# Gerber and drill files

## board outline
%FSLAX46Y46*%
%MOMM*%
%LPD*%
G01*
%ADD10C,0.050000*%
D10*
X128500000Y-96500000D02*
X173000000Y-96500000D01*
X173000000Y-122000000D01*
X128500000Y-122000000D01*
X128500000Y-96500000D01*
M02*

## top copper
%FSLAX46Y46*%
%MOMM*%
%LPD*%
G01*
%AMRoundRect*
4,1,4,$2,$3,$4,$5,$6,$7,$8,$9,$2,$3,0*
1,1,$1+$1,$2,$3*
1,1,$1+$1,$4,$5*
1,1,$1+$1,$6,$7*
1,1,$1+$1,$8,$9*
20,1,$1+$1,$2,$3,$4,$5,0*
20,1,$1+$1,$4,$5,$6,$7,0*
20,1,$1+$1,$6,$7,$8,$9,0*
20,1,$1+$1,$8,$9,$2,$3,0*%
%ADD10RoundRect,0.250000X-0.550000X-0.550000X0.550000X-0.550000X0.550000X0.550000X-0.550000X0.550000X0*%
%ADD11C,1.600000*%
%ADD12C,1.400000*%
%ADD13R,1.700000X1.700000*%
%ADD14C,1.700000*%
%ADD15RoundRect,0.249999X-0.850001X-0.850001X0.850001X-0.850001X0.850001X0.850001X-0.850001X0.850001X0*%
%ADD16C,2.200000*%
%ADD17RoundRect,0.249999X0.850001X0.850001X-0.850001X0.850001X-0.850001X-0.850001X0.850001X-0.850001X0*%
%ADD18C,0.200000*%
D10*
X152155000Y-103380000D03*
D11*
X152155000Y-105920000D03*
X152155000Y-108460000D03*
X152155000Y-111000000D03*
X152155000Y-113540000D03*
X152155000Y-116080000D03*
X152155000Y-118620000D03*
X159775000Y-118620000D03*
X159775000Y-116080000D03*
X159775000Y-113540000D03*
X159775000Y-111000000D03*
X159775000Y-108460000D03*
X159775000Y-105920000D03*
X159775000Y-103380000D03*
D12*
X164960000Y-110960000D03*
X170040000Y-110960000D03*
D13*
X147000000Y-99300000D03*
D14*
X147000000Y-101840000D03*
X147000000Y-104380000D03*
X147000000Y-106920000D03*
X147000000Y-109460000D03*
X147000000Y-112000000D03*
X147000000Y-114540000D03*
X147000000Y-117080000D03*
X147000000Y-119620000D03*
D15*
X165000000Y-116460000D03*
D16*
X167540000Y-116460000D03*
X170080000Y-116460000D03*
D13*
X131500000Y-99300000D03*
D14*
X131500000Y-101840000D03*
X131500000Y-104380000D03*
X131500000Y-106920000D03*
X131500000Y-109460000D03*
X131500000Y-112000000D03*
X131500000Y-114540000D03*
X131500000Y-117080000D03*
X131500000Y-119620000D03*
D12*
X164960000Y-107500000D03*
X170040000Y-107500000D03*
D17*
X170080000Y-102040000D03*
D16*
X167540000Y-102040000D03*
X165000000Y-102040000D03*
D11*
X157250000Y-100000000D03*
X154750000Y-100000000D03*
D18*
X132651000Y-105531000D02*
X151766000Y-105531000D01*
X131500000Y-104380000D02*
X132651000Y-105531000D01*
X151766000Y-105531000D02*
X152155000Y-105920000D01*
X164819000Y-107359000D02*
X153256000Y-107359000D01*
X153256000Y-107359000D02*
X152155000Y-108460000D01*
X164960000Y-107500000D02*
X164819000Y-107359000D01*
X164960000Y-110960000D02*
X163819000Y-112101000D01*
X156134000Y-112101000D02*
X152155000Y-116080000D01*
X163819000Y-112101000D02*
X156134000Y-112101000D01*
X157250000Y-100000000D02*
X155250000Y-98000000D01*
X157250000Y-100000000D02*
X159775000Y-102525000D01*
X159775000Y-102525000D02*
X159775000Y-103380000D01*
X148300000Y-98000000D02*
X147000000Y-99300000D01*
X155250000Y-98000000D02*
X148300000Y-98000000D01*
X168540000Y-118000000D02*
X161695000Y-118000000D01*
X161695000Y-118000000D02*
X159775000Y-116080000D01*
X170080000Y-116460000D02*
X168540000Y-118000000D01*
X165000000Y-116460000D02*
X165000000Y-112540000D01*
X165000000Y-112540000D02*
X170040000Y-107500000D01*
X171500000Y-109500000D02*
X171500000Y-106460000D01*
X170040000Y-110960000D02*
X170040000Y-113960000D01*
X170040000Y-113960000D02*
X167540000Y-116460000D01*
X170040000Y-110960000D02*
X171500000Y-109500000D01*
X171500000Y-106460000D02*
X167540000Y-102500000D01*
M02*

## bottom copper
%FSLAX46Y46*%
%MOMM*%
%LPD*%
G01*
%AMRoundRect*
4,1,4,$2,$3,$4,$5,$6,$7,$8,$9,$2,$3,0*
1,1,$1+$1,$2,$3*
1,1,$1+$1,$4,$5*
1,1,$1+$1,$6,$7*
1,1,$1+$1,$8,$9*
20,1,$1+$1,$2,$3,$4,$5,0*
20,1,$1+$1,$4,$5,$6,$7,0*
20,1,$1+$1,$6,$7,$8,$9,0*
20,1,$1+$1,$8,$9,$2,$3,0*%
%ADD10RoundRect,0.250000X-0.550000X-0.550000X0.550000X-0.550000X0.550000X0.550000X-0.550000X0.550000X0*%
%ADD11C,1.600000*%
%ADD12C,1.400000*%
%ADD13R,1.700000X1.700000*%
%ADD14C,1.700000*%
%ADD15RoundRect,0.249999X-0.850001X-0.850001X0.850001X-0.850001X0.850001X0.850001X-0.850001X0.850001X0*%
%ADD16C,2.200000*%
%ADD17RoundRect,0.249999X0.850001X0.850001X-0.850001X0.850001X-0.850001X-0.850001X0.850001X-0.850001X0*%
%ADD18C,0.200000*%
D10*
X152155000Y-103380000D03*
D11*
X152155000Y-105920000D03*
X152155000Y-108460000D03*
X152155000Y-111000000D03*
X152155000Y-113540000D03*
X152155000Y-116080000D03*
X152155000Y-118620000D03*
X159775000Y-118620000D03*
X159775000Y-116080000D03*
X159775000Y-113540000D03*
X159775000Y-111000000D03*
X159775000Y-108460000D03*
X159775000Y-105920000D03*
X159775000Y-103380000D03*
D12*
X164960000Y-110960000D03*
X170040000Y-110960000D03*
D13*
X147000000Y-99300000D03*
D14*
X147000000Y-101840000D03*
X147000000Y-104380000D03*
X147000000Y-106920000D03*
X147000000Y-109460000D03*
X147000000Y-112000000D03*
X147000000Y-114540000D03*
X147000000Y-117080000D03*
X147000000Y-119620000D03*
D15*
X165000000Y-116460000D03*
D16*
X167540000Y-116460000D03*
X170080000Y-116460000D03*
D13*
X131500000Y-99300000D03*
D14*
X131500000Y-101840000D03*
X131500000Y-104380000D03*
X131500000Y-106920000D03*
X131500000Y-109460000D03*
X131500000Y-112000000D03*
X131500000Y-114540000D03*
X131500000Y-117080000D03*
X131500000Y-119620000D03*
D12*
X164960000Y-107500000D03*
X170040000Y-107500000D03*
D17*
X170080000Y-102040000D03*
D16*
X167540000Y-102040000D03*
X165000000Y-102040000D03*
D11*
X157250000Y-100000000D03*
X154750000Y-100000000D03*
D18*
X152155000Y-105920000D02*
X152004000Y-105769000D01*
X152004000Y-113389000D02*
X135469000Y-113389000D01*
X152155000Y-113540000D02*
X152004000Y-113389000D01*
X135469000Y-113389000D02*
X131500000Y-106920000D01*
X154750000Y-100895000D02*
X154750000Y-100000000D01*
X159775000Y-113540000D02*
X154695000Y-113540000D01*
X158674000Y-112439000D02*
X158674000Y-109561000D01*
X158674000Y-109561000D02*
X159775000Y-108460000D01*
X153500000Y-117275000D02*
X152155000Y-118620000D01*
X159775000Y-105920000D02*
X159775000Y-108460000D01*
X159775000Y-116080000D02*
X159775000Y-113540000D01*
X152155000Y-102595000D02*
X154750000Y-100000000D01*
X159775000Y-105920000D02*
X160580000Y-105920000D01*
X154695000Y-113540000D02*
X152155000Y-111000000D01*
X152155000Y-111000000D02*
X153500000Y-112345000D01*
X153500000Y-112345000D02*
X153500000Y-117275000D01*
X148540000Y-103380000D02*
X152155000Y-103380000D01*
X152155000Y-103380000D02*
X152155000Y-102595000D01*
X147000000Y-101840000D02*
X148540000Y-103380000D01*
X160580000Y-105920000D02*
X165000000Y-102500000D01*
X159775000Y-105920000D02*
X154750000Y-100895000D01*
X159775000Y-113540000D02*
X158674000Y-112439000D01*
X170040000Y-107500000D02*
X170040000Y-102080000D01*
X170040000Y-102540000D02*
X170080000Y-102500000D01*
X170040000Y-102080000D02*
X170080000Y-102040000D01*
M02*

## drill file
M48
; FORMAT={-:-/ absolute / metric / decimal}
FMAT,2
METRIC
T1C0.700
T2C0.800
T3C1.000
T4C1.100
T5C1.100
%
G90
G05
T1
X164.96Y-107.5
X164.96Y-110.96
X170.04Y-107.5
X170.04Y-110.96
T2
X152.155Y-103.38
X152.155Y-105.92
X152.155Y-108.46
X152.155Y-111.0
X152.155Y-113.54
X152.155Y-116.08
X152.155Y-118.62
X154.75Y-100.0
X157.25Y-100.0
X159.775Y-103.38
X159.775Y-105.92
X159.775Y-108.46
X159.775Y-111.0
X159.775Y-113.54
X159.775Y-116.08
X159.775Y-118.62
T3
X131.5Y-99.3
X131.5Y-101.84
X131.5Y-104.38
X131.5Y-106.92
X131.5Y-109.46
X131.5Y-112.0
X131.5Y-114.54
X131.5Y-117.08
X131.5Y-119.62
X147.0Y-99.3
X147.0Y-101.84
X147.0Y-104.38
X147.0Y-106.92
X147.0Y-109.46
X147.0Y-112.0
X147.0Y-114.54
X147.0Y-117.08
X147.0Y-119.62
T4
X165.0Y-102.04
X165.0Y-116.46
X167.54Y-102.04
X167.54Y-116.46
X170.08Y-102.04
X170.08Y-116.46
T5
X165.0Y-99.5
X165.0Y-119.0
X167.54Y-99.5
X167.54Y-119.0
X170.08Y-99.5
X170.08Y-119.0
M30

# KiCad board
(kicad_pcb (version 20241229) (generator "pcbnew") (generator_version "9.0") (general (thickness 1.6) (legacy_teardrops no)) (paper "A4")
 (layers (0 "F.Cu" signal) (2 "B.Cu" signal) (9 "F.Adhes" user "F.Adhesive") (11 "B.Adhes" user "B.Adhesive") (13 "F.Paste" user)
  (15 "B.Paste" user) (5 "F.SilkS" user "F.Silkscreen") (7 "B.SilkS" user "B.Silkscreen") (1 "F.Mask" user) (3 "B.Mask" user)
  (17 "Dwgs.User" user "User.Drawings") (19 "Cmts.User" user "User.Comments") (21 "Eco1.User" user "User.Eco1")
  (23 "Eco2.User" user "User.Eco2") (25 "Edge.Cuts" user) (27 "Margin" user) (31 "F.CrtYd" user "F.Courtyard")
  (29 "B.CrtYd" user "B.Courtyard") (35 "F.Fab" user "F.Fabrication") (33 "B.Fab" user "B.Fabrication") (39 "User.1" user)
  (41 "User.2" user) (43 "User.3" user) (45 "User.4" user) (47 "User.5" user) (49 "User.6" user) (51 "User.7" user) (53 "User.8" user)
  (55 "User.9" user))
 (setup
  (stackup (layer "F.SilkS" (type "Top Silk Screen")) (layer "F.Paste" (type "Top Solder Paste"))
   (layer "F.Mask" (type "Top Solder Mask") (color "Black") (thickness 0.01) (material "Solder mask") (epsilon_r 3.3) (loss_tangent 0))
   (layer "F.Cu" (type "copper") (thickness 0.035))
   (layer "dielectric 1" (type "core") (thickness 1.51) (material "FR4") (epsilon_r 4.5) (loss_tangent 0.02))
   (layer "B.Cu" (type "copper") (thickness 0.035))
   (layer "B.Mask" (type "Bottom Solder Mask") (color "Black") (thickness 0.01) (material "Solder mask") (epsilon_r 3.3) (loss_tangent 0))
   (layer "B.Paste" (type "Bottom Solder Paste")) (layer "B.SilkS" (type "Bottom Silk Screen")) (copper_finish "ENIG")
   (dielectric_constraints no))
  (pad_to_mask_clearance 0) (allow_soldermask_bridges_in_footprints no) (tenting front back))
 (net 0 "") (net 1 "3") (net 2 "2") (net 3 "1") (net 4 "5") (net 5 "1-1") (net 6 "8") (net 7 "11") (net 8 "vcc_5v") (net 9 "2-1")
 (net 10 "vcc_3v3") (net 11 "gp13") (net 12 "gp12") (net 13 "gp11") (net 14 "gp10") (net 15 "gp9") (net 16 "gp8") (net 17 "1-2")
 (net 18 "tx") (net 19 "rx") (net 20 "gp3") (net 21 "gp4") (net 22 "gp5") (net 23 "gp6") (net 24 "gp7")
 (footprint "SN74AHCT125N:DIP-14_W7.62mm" (layer "F.Cu") (at 152.155 103.38)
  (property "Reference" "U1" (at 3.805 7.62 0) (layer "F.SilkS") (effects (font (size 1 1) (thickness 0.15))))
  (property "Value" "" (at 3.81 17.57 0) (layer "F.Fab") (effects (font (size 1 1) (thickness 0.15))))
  (pad "1" thru_hole roundrect (at 0 0) (size 1.6 1.6) (drill 0.8) (layers "*.Cu" "*.Mask") (remove_unused_layers no)
   (roundrect_rratio 0.15625) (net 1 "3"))
  (pad "2" thru_hole circle (at 0 2.54) (size 1.6 1.6) (drill 0.8) (layers "*.Cu" "*.Mask") (remove_unused_layers no) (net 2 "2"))
  (pad "3" thru_hole circle (at 0 5.08) (size 1.6 1.6) (drill 0.8) (layers "*.Cu" "*.Mask") (remove_unused_layers no) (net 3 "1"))
  (pad "4" thru_hole circle (at 0 7.62) (size 1.6 1.6) (drill 0.8) (layers "*.Cu" "*.Mask") (remove_unused_layers no) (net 1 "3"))
  (pad "5" thru_hole circle (at 0 10.16) (size 1.6 1.6) (drill 0.8) (layers "*.Cu" "*.Mask") (remove_unused_layers no) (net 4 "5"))
  (pad "6" thru_hole circle (at 0 12.7) (size 1.6 1.6) (drill 0.8) (layers "*.Cu" "*.Mask") (remove_unused_layers no) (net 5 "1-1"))
  (pad "7" thru_hole circle (at 0 15.24) (size 1.6 1.6) (drill 0.8) (layers "*.Cu" "*.Mask") (remove_unused_layers no) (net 1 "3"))
  (pad "8" thru_hole circle (at 7.62 15.24) (size 1.6 1.6) (drill 0.8) (layers "*.Cu" "*.Mask") (remove_unused_layers no) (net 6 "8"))
  (pad "9" thru_hole circle (at 7.62 12.7) (size 1.6 1.6) (drill 0.8) (layers "*.Cu" "*.Mask") (remove_unused_layers no) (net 1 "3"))
  (pad "10" thru_hole circle (at 7.62 10.16) (size 1.6 1.6) (drill 0.8) (layers "*.Cu" "*.Mask") (remove_unused_layers no) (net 1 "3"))
  (pad "11" thru_hole circle (at 7.62 7.62) (size 1.6 1.6) (drill 0.8) (layers "*.Cu" "*.Mask") (remove_unused_layers no) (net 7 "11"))
  (pad "12" thru_hole circle (at 7.62 5.08) (size 1.6 1.6) (drill 0.8) (layers "*.Cu" "*.Mask") (remove_unused_layers no) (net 1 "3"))
  (pad "13" thru_hole circle (at 7.62 2.54) (size 1.6 1.6) (drill 0.8) (layers "*.Cu" "*.Mask") (remove_unused_layers no) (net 1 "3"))
  (pad "14" thru_hole circle (at 7.62 0) (size 1.6 1.6) (drill 0.8) (layers "*.Cu" "*.Mask") (remove_unused_layers no) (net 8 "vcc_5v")))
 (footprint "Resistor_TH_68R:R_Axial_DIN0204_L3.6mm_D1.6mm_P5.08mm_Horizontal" (layer "F.Cu") (at 164.96 110.96)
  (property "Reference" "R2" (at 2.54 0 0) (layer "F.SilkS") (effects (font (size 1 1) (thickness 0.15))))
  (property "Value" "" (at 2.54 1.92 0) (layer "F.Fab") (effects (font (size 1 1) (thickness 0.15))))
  (pad "1" thru_hole circle (at 0 0) (size 1.4 1.4) (drill 0.7) (layers "*.Cu" "*.Mask") (remove_unused_layers no) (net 5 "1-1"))
  (pad "2" thru_hole circle (at 5.08 0) (size 1.4 1.4) (drill 0.7) (layers "*.Cu" "*.Mask") (remove_unused_layers no) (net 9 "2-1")))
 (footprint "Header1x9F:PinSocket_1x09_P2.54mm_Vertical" (layer "F.Cu") (at 147 99.3)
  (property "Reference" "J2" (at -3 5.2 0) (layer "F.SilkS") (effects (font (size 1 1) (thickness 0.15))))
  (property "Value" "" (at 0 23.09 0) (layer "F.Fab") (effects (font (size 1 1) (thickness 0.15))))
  (pad "1" thru_hole rect (at 0 0) (size 1.7 1.7) (drill 1) (layers "*.Cu" "*.Mask") (remove_unused_layers no) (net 8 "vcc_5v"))
  (pad "2" thru_hole circle (at 0 2.54) (size 1.7 1.7) (drill 1) (layers "*.Cu" "*.Mask") (remove_unused_layers no) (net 1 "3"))
  (pad "3" thru_hole circle (at 0 5.08) (size 1.7 1.7) (drill 1) (layers "*.Cu" "*.Mask") (remove_unused_layers no) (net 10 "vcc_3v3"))
  (pad "4" thru_hole circle (at 0 7.62) (size 1.7 1.7) (drill 1) (layers "*.Cu" "*.Mask") (remove_unused_layers no) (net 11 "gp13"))
  (pad "5" thru_hole circle (at 0 10.16) (size 1.7 1.7) (drill 1) (layers "*.Cu" "*.Mask") (remove_unused_layers no) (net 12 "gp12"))
  (pad "6" thru_hole circle (at 0 12.7) (size 1.7 1.7) (drill 1) (layers "*.Cu" "*.Mask") (remove_unused_layers no) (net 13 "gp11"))
  (pad "7" thru_hole circle (at 0 15.24) (size 1.7 1.7) (drill 1) (layers "*.Cu" "*.Mask") (remove_unused_layers no) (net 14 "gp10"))
  (pad "8" thru_hole circle (at 0 17.78) (size 1.7 1.7) (drill 1) (layers "*.Cu" "*.Mask") (remove_unused_layers no) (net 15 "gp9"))
  (pad "9" thru_hole circle (at 0 20.32) (size 1.7 1.7) (drill 1) (layers "*.Cu" "*.Mask") (remove_unused_layers no) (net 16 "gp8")))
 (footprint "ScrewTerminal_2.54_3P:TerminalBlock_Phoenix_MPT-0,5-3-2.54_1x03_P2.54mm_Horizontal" (layer "F.Cu") (at 165 116.46)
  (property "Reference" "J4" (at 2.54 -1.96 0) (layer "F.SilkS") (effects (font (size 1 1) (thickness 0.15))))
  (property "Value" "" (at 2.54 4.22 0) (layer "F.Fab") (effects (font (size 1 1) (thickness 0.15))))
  (pad "" np_thru_hole circle (at 0 2.54) (size 1.1 1.1) (drill 1.1) (layers "*.Cu" "*.Mask"))
  (pad "" np_thru_hole circle (at 2.54 2.54) (size 1.1 1.1) (drill 1.1) (layers "*.Cu" "*.Mask"))
  (pad "" np_thru_hole circle (at 5.08 2.54) (size 1.1 1.1) (drill 1.1) (layers "*.Cu" "*.Mask"))
  (pad "1" thru_hole roundrect (at 0 0) (size 2.2 2.2) (drill 1.1) (layers "*.Cu" "*.Mask") (remove_unused_layers no)
   (roundrect_rratio 0.113636) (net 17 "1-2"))
  (pad "2" thru_hole circle (at 2.54 0) (size 2.2 2.2) (drill 1.1) (layers "*.Cu" "*.Mask") (remove_unused_layers no) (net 9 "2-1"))
  (pad "3" thru_hole circle (at 5.08 0) (size 2.2 2.2) (drill 1.1) (layers "*.Cu" "*.Mask") (remove_unused_layers no) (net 1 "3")))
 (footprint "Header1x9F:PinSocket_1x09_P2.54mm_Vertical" (layer "F.Cu") (at 131.5 99.3)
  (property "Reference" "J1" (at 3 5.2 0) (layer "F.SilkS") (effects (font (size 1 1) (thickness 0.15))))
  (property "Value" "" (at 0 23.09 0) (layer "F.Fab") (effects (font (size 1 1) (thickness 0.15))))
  (pad "1" thru_hole rect (at 0 0) (size 1.7 1.7) (drill 1) (layers "*.Cu" "*.Mask") (remove_unused_layers no) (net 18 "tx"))
  (pad "2" thru_hole circle (at 0 2.54) (size 1.7 1.7) (drill 1) (layers "*.Cu" "*.Mask") (remove_unused_layers no) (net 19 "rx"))
  (pad "3" thru_hole circle (at 0 5.08) (size 1.7 1.7) (drill 1) (layers "*.Cu" "*.Mask") (remove_unused_layers no) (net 2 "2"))
  (pad "4" thru_hole circle (at 0 7.62) (size 1.7 1.7) (drill 1) (layers "*.Cu" "*.Mask") (remove_unused_layers no) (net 4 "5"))
  (pad "5" thru_hole circle (at 0 10.16) (size 1.7 1.7) (drill 1) (layers "*.Cu" "*.Mask") (remove_unused_layers no) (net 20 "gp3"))
  (pad "6" thru_hole circle (at 0 12.7) (size 1.7 1.7) (drill 1) (layers "*.Cu" "*.Mask") (remove_unused_layers no) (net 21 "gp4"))
  (pad "7" thru_hole circle (at 0 15.24) (size 1.7 1.7) (drill 1) (layers "*.Cu" "*.Mask") (remove_unused_layers no) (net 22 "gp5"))
  (pad "8" thru_hole circle (at 0 17.78) (size 1.7 1.7) (drill 1) (layers "*.Cu" "*.Mask") (remove_unused_layers no) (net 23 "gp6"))
  (pad "9" thru_hole circle (at 0 20.32) (size 1.7 1.7) (drill 1) (layers "*.Cu" "*.Mask") (remove_unused_layers no) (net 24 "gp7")))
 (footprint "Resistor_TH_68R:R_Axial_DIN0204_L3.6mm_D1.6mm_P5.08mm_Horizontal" (layer "F.Cu") (at 164.96 107.5)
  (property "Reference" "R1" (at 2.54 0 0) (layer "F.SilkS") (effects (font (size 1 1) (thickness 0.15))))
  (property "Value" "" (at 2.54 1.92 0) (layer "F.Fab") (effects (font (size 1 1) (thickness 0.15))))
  (pad "1" thru_hole circle (at 0 0) (size 1.4 1.4) (drill 0.7) (layers "*.Cu" "*.Mask") (remove_unused_layers no) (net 3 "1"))
  (pad "2" thru_hole circle (at 5.08 0) (size 1.4 1.4) (drill 0.7) (layers "*.Cu" "*.Mask") (remove_unused_layers no) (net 17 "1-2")))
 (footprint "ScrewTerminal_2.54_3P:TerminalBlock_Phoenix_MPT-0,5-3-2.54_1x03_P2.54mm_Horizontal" (layer "F.Cu") (at 170.08 102.04 180)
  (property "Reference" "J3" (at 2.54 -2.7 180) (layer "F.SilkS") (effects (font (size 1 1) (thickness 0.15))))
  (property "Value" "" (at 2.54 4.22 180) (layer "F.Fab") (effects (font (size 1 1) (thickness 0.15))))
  (pad "" np_thru_hole circle (at 0 2.54 180) (size 1.1 1.1) (drill 1.1) (layers "*.Cu" "*.Mask"))
  (pad "" np_thru_hole circle (at 2.54 2.54 180) (size 1.1 1.1) (drill 1.1) (layers "*.Cu" "*.Mask"))
  (pad "" np_thru_hole circle (at 5.08 2.54 180) (size 1.1 1.1) (drill 1.1) (layers "*.Cu" "*.Mask"))
  (pad "1" thru_hole roundrect (at 0 0 180) (size 2.2 2.2) (drill 1.1) (layers "*.Cu" "*.Mask") (remove_unused_layers no)
   (roundrect_rratio 0.113636) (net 17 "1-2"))
  (pad "2" thru_hole circle (at 2.54 0 180) (size 2.2 2.2) (drill 1.1) (layers "*.Cu" "*.Mask") (remove_unused_layers no) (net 9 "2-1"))
  (pad "3" thru_hole circle (at 5.08 0 180) (size 2.2 2.2) (drill 1.1) (layers "*.Cu" "*.Mask") (remove_unused_layers no) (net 1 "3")))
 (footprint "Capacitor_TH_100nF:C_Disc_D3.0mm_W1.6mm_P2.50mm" (layer "F.Cu") (at 157.25 100 180)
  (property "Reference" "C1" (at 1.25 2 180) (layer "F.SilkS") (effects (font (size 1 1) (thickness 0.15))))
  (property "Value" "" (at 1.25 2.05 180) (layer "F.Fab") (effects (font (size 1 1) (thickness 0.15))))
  (pad "1" thru_hole circle (at 0 0 180) (size 1.6 1.6) (drill 0.8) (layers "*.Cu" "*.Mask") (remove_unused_layers no) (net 8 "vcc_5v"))
  (pad "2" thru_hole circle (at 2.5 0 180) (size 1.6 1.6) (drill 0.8) (layers "*.Cu" "*.Mask") (remove_unused_layers no) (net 1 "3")))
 (gr_rect (start 128.5 96.5) (end 173 122) (stroke (width 0.05) (type default)) (fill no) (layer "Edge.Cuts"))
 (segment (start 132.651 105.531) (end 151.766 105.531) (width 0.2) (layer "F.Cu") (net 2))
 (segment (start 131.5 104.38) (end 132.651 105.531) (width 0.2) (layer "F.Cu") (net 2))
 (segment (start 151.766 105.531) (end 152.155 105.92) (width 0.2) (layer "F.Cu") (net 2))
 (segment (start 152.155 105.92) (end 152.004 105.769) (width 0.2) (layer "B.Cu") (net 2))
 (segment (start 152.004 113.389) (end 135.469 113.389) (width 0.2) (layer "B.Cu") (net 4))
 (segment (start 152.155 113.54) (end 152.004 113.389) (width 0.2) (layer "B.Cu") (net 4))
 (segment (start 135.469 113.389) (end 131.5 106.92) (width 0.2) (layer "B.Cu") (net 4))
 (segment (start 164.819 107.359) (end 153.256 107.359) (width 0.2) (layer "F.Cu") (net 3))
 (segment (start 153.256 107.359) (end 152.155 108.46) (width 0.2) (layer "F.Cu") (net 3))
 (segment (start 164.96 107.5) (end 164.819 107.359) (width 0.2) (layer "F.Cu") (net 3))
 (segment (start 164.96 110.96) (end 163.819 112.101) (width 0.2) (layer "F.Cu") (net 5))
 (segment (start 156.134 112.101) (end 152.155 116.08) (width 0.2) (layer "F.Cu") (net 5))
 (segment (start 163.819 112.101) (end 156.134 112.101) (width 0.2) (layer "F.Cu") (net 5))
 (segment (start 157.25 100) (end 155.25 98) (width 0.2) (layer "F.Cu") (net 8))
 (segment (start 157.25 100) (end 159.775 102.525) (width 0.2) (layer "F.Cu") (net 8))
 (segment (start 159.775 102.525) (end 159.775 103.38) (width 0.2) (layer "F.Cu") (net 8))
 (segment (start 148.3 98) (end 147 99.3) (width 0.2) (layer "F.Cu") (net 8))
 (segment (start 155.25 98) (end 148.3 98) (width 0.2) (layer "F.Cu") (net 8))
 (segment (start 168.54 118) (end 161.695 118) (width 0.2) (layer "F.Cu") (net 1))
 (segment (start 161.695 118) (end 159.775 116.08) (width 0.2) (layer "F.Cu") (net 1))
 (segment (start 170.08 116.46) (end 168.54 118) (width 0.2) (layer "F.Cu") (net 1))
 (segment (start 154.75 100.895) (end 154.75 100) (width 0.2) (layer "B.Cu") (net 1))
 (segment (start 159.775 113.54) (end 154.695 113.54) (width 0.2) (layer "B.Cu") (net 1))
 (segment (start 158.674 112.439) (end 158.674 109.561) (width 0.2) (layer "B.Cu") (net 1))
 (segment (start 158.674 109.561) (end 159.775 108.46) (width 0.2) (layer "B.Cu") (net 1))
 (segment (start 153.5 117.275) (end 152.155 118.62) (width 0.2) (layer "B.Cu") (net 1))
 (segment (start 159.775 105.92) (end 159.775 108.46) (width 0.2) (layer "B.Cu") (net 1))
 (segment (start 159.775 116.08) (end 159.775 113.54) (width 0.2) (layer "B.Cu") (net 1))
 (segment (start 152.155 102.595) (end 154.75 100) (width 0.2) (layer "B.Cu") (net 1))
 (segment (start 159.775 105.92) (end 160.58 105.92) (width 0.2) (layer "B.Cu") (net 1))
 (segment (start 154.695 113.54) (end 152.155 111) (width 0.2) (layer "B.Cu") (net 1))
 (segment (start 152.155 111) (end 153.5 112.345) (width 0.2) (layer "B.Cu") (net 1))
 (segment (start 153.5 112.345) (end 153.5 117.275) (width 0.2) (layer "B.Cu") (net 1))
 (segment (start 148.54 103.38) (end 152.155 103.38) (width 0.2) (layer "B.Cu") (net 1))
 (segment (start 152.155 103.38) (end 152.155 102.595) (width 0.2) (layer "B.Cu") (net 1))
 (segment (start 147 101.84) (end 148.54 103.38) (width 0.2) (layer "B.Cu") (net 1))
 (segment (start 160.58 105.92) (end 165 102.5) (width 0.2) (layer "B.Cu") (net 1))
 (segment (start 159.775 105.92) (end 154.75 100.895) (width 0.2) (layer "B.Cu") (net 1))
 (segment (start 159.775 113.54) (end 158.674 112.439) (width 0.2) (layer "B.Cu") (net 1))
 (segment (start 165 116.46) (end 165 112.54) (width 0.2) (layer "F.Cu") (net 17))
 (segment (start 165 112.54) (end 170.04 107.5) (width 0.2) (layer "F.Cu") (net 17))
 (segment (start 170.04 107.5) (end 170.04 102.08) (width 0.2) (layer "B.Cu") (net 17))
 (segment (start 170.04 102.54) (end 170.08 102.5) (width 0.2) (layer "B.Cu") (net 17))
 (segment (start 170.04 102.08) (end 170.08 102.04) (width 0.2) (layer "B.Cu") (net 17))
 (segment (start 171.5 109.5) (end 171.5 106.46) (width 0.2) (layer "F.Cu") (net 9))
 (segment (start 170.04 110.96) (end 170.04 113.96) (width 0.2) (layer "F.Cu") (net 9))
 (segment (start 170.04 113.96) (end 167.54 116.46) (width 0.2) (layer "F.Cu") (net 9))
 (segment (start 170.04 110.96) (end 171.5 109.5) (width 0.2) (layer "F.Cu") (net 9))
 (segment (start 171.5 106.46) (end 167.54 102.5) (width 0.2) (layer "F.Cu") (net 9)))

